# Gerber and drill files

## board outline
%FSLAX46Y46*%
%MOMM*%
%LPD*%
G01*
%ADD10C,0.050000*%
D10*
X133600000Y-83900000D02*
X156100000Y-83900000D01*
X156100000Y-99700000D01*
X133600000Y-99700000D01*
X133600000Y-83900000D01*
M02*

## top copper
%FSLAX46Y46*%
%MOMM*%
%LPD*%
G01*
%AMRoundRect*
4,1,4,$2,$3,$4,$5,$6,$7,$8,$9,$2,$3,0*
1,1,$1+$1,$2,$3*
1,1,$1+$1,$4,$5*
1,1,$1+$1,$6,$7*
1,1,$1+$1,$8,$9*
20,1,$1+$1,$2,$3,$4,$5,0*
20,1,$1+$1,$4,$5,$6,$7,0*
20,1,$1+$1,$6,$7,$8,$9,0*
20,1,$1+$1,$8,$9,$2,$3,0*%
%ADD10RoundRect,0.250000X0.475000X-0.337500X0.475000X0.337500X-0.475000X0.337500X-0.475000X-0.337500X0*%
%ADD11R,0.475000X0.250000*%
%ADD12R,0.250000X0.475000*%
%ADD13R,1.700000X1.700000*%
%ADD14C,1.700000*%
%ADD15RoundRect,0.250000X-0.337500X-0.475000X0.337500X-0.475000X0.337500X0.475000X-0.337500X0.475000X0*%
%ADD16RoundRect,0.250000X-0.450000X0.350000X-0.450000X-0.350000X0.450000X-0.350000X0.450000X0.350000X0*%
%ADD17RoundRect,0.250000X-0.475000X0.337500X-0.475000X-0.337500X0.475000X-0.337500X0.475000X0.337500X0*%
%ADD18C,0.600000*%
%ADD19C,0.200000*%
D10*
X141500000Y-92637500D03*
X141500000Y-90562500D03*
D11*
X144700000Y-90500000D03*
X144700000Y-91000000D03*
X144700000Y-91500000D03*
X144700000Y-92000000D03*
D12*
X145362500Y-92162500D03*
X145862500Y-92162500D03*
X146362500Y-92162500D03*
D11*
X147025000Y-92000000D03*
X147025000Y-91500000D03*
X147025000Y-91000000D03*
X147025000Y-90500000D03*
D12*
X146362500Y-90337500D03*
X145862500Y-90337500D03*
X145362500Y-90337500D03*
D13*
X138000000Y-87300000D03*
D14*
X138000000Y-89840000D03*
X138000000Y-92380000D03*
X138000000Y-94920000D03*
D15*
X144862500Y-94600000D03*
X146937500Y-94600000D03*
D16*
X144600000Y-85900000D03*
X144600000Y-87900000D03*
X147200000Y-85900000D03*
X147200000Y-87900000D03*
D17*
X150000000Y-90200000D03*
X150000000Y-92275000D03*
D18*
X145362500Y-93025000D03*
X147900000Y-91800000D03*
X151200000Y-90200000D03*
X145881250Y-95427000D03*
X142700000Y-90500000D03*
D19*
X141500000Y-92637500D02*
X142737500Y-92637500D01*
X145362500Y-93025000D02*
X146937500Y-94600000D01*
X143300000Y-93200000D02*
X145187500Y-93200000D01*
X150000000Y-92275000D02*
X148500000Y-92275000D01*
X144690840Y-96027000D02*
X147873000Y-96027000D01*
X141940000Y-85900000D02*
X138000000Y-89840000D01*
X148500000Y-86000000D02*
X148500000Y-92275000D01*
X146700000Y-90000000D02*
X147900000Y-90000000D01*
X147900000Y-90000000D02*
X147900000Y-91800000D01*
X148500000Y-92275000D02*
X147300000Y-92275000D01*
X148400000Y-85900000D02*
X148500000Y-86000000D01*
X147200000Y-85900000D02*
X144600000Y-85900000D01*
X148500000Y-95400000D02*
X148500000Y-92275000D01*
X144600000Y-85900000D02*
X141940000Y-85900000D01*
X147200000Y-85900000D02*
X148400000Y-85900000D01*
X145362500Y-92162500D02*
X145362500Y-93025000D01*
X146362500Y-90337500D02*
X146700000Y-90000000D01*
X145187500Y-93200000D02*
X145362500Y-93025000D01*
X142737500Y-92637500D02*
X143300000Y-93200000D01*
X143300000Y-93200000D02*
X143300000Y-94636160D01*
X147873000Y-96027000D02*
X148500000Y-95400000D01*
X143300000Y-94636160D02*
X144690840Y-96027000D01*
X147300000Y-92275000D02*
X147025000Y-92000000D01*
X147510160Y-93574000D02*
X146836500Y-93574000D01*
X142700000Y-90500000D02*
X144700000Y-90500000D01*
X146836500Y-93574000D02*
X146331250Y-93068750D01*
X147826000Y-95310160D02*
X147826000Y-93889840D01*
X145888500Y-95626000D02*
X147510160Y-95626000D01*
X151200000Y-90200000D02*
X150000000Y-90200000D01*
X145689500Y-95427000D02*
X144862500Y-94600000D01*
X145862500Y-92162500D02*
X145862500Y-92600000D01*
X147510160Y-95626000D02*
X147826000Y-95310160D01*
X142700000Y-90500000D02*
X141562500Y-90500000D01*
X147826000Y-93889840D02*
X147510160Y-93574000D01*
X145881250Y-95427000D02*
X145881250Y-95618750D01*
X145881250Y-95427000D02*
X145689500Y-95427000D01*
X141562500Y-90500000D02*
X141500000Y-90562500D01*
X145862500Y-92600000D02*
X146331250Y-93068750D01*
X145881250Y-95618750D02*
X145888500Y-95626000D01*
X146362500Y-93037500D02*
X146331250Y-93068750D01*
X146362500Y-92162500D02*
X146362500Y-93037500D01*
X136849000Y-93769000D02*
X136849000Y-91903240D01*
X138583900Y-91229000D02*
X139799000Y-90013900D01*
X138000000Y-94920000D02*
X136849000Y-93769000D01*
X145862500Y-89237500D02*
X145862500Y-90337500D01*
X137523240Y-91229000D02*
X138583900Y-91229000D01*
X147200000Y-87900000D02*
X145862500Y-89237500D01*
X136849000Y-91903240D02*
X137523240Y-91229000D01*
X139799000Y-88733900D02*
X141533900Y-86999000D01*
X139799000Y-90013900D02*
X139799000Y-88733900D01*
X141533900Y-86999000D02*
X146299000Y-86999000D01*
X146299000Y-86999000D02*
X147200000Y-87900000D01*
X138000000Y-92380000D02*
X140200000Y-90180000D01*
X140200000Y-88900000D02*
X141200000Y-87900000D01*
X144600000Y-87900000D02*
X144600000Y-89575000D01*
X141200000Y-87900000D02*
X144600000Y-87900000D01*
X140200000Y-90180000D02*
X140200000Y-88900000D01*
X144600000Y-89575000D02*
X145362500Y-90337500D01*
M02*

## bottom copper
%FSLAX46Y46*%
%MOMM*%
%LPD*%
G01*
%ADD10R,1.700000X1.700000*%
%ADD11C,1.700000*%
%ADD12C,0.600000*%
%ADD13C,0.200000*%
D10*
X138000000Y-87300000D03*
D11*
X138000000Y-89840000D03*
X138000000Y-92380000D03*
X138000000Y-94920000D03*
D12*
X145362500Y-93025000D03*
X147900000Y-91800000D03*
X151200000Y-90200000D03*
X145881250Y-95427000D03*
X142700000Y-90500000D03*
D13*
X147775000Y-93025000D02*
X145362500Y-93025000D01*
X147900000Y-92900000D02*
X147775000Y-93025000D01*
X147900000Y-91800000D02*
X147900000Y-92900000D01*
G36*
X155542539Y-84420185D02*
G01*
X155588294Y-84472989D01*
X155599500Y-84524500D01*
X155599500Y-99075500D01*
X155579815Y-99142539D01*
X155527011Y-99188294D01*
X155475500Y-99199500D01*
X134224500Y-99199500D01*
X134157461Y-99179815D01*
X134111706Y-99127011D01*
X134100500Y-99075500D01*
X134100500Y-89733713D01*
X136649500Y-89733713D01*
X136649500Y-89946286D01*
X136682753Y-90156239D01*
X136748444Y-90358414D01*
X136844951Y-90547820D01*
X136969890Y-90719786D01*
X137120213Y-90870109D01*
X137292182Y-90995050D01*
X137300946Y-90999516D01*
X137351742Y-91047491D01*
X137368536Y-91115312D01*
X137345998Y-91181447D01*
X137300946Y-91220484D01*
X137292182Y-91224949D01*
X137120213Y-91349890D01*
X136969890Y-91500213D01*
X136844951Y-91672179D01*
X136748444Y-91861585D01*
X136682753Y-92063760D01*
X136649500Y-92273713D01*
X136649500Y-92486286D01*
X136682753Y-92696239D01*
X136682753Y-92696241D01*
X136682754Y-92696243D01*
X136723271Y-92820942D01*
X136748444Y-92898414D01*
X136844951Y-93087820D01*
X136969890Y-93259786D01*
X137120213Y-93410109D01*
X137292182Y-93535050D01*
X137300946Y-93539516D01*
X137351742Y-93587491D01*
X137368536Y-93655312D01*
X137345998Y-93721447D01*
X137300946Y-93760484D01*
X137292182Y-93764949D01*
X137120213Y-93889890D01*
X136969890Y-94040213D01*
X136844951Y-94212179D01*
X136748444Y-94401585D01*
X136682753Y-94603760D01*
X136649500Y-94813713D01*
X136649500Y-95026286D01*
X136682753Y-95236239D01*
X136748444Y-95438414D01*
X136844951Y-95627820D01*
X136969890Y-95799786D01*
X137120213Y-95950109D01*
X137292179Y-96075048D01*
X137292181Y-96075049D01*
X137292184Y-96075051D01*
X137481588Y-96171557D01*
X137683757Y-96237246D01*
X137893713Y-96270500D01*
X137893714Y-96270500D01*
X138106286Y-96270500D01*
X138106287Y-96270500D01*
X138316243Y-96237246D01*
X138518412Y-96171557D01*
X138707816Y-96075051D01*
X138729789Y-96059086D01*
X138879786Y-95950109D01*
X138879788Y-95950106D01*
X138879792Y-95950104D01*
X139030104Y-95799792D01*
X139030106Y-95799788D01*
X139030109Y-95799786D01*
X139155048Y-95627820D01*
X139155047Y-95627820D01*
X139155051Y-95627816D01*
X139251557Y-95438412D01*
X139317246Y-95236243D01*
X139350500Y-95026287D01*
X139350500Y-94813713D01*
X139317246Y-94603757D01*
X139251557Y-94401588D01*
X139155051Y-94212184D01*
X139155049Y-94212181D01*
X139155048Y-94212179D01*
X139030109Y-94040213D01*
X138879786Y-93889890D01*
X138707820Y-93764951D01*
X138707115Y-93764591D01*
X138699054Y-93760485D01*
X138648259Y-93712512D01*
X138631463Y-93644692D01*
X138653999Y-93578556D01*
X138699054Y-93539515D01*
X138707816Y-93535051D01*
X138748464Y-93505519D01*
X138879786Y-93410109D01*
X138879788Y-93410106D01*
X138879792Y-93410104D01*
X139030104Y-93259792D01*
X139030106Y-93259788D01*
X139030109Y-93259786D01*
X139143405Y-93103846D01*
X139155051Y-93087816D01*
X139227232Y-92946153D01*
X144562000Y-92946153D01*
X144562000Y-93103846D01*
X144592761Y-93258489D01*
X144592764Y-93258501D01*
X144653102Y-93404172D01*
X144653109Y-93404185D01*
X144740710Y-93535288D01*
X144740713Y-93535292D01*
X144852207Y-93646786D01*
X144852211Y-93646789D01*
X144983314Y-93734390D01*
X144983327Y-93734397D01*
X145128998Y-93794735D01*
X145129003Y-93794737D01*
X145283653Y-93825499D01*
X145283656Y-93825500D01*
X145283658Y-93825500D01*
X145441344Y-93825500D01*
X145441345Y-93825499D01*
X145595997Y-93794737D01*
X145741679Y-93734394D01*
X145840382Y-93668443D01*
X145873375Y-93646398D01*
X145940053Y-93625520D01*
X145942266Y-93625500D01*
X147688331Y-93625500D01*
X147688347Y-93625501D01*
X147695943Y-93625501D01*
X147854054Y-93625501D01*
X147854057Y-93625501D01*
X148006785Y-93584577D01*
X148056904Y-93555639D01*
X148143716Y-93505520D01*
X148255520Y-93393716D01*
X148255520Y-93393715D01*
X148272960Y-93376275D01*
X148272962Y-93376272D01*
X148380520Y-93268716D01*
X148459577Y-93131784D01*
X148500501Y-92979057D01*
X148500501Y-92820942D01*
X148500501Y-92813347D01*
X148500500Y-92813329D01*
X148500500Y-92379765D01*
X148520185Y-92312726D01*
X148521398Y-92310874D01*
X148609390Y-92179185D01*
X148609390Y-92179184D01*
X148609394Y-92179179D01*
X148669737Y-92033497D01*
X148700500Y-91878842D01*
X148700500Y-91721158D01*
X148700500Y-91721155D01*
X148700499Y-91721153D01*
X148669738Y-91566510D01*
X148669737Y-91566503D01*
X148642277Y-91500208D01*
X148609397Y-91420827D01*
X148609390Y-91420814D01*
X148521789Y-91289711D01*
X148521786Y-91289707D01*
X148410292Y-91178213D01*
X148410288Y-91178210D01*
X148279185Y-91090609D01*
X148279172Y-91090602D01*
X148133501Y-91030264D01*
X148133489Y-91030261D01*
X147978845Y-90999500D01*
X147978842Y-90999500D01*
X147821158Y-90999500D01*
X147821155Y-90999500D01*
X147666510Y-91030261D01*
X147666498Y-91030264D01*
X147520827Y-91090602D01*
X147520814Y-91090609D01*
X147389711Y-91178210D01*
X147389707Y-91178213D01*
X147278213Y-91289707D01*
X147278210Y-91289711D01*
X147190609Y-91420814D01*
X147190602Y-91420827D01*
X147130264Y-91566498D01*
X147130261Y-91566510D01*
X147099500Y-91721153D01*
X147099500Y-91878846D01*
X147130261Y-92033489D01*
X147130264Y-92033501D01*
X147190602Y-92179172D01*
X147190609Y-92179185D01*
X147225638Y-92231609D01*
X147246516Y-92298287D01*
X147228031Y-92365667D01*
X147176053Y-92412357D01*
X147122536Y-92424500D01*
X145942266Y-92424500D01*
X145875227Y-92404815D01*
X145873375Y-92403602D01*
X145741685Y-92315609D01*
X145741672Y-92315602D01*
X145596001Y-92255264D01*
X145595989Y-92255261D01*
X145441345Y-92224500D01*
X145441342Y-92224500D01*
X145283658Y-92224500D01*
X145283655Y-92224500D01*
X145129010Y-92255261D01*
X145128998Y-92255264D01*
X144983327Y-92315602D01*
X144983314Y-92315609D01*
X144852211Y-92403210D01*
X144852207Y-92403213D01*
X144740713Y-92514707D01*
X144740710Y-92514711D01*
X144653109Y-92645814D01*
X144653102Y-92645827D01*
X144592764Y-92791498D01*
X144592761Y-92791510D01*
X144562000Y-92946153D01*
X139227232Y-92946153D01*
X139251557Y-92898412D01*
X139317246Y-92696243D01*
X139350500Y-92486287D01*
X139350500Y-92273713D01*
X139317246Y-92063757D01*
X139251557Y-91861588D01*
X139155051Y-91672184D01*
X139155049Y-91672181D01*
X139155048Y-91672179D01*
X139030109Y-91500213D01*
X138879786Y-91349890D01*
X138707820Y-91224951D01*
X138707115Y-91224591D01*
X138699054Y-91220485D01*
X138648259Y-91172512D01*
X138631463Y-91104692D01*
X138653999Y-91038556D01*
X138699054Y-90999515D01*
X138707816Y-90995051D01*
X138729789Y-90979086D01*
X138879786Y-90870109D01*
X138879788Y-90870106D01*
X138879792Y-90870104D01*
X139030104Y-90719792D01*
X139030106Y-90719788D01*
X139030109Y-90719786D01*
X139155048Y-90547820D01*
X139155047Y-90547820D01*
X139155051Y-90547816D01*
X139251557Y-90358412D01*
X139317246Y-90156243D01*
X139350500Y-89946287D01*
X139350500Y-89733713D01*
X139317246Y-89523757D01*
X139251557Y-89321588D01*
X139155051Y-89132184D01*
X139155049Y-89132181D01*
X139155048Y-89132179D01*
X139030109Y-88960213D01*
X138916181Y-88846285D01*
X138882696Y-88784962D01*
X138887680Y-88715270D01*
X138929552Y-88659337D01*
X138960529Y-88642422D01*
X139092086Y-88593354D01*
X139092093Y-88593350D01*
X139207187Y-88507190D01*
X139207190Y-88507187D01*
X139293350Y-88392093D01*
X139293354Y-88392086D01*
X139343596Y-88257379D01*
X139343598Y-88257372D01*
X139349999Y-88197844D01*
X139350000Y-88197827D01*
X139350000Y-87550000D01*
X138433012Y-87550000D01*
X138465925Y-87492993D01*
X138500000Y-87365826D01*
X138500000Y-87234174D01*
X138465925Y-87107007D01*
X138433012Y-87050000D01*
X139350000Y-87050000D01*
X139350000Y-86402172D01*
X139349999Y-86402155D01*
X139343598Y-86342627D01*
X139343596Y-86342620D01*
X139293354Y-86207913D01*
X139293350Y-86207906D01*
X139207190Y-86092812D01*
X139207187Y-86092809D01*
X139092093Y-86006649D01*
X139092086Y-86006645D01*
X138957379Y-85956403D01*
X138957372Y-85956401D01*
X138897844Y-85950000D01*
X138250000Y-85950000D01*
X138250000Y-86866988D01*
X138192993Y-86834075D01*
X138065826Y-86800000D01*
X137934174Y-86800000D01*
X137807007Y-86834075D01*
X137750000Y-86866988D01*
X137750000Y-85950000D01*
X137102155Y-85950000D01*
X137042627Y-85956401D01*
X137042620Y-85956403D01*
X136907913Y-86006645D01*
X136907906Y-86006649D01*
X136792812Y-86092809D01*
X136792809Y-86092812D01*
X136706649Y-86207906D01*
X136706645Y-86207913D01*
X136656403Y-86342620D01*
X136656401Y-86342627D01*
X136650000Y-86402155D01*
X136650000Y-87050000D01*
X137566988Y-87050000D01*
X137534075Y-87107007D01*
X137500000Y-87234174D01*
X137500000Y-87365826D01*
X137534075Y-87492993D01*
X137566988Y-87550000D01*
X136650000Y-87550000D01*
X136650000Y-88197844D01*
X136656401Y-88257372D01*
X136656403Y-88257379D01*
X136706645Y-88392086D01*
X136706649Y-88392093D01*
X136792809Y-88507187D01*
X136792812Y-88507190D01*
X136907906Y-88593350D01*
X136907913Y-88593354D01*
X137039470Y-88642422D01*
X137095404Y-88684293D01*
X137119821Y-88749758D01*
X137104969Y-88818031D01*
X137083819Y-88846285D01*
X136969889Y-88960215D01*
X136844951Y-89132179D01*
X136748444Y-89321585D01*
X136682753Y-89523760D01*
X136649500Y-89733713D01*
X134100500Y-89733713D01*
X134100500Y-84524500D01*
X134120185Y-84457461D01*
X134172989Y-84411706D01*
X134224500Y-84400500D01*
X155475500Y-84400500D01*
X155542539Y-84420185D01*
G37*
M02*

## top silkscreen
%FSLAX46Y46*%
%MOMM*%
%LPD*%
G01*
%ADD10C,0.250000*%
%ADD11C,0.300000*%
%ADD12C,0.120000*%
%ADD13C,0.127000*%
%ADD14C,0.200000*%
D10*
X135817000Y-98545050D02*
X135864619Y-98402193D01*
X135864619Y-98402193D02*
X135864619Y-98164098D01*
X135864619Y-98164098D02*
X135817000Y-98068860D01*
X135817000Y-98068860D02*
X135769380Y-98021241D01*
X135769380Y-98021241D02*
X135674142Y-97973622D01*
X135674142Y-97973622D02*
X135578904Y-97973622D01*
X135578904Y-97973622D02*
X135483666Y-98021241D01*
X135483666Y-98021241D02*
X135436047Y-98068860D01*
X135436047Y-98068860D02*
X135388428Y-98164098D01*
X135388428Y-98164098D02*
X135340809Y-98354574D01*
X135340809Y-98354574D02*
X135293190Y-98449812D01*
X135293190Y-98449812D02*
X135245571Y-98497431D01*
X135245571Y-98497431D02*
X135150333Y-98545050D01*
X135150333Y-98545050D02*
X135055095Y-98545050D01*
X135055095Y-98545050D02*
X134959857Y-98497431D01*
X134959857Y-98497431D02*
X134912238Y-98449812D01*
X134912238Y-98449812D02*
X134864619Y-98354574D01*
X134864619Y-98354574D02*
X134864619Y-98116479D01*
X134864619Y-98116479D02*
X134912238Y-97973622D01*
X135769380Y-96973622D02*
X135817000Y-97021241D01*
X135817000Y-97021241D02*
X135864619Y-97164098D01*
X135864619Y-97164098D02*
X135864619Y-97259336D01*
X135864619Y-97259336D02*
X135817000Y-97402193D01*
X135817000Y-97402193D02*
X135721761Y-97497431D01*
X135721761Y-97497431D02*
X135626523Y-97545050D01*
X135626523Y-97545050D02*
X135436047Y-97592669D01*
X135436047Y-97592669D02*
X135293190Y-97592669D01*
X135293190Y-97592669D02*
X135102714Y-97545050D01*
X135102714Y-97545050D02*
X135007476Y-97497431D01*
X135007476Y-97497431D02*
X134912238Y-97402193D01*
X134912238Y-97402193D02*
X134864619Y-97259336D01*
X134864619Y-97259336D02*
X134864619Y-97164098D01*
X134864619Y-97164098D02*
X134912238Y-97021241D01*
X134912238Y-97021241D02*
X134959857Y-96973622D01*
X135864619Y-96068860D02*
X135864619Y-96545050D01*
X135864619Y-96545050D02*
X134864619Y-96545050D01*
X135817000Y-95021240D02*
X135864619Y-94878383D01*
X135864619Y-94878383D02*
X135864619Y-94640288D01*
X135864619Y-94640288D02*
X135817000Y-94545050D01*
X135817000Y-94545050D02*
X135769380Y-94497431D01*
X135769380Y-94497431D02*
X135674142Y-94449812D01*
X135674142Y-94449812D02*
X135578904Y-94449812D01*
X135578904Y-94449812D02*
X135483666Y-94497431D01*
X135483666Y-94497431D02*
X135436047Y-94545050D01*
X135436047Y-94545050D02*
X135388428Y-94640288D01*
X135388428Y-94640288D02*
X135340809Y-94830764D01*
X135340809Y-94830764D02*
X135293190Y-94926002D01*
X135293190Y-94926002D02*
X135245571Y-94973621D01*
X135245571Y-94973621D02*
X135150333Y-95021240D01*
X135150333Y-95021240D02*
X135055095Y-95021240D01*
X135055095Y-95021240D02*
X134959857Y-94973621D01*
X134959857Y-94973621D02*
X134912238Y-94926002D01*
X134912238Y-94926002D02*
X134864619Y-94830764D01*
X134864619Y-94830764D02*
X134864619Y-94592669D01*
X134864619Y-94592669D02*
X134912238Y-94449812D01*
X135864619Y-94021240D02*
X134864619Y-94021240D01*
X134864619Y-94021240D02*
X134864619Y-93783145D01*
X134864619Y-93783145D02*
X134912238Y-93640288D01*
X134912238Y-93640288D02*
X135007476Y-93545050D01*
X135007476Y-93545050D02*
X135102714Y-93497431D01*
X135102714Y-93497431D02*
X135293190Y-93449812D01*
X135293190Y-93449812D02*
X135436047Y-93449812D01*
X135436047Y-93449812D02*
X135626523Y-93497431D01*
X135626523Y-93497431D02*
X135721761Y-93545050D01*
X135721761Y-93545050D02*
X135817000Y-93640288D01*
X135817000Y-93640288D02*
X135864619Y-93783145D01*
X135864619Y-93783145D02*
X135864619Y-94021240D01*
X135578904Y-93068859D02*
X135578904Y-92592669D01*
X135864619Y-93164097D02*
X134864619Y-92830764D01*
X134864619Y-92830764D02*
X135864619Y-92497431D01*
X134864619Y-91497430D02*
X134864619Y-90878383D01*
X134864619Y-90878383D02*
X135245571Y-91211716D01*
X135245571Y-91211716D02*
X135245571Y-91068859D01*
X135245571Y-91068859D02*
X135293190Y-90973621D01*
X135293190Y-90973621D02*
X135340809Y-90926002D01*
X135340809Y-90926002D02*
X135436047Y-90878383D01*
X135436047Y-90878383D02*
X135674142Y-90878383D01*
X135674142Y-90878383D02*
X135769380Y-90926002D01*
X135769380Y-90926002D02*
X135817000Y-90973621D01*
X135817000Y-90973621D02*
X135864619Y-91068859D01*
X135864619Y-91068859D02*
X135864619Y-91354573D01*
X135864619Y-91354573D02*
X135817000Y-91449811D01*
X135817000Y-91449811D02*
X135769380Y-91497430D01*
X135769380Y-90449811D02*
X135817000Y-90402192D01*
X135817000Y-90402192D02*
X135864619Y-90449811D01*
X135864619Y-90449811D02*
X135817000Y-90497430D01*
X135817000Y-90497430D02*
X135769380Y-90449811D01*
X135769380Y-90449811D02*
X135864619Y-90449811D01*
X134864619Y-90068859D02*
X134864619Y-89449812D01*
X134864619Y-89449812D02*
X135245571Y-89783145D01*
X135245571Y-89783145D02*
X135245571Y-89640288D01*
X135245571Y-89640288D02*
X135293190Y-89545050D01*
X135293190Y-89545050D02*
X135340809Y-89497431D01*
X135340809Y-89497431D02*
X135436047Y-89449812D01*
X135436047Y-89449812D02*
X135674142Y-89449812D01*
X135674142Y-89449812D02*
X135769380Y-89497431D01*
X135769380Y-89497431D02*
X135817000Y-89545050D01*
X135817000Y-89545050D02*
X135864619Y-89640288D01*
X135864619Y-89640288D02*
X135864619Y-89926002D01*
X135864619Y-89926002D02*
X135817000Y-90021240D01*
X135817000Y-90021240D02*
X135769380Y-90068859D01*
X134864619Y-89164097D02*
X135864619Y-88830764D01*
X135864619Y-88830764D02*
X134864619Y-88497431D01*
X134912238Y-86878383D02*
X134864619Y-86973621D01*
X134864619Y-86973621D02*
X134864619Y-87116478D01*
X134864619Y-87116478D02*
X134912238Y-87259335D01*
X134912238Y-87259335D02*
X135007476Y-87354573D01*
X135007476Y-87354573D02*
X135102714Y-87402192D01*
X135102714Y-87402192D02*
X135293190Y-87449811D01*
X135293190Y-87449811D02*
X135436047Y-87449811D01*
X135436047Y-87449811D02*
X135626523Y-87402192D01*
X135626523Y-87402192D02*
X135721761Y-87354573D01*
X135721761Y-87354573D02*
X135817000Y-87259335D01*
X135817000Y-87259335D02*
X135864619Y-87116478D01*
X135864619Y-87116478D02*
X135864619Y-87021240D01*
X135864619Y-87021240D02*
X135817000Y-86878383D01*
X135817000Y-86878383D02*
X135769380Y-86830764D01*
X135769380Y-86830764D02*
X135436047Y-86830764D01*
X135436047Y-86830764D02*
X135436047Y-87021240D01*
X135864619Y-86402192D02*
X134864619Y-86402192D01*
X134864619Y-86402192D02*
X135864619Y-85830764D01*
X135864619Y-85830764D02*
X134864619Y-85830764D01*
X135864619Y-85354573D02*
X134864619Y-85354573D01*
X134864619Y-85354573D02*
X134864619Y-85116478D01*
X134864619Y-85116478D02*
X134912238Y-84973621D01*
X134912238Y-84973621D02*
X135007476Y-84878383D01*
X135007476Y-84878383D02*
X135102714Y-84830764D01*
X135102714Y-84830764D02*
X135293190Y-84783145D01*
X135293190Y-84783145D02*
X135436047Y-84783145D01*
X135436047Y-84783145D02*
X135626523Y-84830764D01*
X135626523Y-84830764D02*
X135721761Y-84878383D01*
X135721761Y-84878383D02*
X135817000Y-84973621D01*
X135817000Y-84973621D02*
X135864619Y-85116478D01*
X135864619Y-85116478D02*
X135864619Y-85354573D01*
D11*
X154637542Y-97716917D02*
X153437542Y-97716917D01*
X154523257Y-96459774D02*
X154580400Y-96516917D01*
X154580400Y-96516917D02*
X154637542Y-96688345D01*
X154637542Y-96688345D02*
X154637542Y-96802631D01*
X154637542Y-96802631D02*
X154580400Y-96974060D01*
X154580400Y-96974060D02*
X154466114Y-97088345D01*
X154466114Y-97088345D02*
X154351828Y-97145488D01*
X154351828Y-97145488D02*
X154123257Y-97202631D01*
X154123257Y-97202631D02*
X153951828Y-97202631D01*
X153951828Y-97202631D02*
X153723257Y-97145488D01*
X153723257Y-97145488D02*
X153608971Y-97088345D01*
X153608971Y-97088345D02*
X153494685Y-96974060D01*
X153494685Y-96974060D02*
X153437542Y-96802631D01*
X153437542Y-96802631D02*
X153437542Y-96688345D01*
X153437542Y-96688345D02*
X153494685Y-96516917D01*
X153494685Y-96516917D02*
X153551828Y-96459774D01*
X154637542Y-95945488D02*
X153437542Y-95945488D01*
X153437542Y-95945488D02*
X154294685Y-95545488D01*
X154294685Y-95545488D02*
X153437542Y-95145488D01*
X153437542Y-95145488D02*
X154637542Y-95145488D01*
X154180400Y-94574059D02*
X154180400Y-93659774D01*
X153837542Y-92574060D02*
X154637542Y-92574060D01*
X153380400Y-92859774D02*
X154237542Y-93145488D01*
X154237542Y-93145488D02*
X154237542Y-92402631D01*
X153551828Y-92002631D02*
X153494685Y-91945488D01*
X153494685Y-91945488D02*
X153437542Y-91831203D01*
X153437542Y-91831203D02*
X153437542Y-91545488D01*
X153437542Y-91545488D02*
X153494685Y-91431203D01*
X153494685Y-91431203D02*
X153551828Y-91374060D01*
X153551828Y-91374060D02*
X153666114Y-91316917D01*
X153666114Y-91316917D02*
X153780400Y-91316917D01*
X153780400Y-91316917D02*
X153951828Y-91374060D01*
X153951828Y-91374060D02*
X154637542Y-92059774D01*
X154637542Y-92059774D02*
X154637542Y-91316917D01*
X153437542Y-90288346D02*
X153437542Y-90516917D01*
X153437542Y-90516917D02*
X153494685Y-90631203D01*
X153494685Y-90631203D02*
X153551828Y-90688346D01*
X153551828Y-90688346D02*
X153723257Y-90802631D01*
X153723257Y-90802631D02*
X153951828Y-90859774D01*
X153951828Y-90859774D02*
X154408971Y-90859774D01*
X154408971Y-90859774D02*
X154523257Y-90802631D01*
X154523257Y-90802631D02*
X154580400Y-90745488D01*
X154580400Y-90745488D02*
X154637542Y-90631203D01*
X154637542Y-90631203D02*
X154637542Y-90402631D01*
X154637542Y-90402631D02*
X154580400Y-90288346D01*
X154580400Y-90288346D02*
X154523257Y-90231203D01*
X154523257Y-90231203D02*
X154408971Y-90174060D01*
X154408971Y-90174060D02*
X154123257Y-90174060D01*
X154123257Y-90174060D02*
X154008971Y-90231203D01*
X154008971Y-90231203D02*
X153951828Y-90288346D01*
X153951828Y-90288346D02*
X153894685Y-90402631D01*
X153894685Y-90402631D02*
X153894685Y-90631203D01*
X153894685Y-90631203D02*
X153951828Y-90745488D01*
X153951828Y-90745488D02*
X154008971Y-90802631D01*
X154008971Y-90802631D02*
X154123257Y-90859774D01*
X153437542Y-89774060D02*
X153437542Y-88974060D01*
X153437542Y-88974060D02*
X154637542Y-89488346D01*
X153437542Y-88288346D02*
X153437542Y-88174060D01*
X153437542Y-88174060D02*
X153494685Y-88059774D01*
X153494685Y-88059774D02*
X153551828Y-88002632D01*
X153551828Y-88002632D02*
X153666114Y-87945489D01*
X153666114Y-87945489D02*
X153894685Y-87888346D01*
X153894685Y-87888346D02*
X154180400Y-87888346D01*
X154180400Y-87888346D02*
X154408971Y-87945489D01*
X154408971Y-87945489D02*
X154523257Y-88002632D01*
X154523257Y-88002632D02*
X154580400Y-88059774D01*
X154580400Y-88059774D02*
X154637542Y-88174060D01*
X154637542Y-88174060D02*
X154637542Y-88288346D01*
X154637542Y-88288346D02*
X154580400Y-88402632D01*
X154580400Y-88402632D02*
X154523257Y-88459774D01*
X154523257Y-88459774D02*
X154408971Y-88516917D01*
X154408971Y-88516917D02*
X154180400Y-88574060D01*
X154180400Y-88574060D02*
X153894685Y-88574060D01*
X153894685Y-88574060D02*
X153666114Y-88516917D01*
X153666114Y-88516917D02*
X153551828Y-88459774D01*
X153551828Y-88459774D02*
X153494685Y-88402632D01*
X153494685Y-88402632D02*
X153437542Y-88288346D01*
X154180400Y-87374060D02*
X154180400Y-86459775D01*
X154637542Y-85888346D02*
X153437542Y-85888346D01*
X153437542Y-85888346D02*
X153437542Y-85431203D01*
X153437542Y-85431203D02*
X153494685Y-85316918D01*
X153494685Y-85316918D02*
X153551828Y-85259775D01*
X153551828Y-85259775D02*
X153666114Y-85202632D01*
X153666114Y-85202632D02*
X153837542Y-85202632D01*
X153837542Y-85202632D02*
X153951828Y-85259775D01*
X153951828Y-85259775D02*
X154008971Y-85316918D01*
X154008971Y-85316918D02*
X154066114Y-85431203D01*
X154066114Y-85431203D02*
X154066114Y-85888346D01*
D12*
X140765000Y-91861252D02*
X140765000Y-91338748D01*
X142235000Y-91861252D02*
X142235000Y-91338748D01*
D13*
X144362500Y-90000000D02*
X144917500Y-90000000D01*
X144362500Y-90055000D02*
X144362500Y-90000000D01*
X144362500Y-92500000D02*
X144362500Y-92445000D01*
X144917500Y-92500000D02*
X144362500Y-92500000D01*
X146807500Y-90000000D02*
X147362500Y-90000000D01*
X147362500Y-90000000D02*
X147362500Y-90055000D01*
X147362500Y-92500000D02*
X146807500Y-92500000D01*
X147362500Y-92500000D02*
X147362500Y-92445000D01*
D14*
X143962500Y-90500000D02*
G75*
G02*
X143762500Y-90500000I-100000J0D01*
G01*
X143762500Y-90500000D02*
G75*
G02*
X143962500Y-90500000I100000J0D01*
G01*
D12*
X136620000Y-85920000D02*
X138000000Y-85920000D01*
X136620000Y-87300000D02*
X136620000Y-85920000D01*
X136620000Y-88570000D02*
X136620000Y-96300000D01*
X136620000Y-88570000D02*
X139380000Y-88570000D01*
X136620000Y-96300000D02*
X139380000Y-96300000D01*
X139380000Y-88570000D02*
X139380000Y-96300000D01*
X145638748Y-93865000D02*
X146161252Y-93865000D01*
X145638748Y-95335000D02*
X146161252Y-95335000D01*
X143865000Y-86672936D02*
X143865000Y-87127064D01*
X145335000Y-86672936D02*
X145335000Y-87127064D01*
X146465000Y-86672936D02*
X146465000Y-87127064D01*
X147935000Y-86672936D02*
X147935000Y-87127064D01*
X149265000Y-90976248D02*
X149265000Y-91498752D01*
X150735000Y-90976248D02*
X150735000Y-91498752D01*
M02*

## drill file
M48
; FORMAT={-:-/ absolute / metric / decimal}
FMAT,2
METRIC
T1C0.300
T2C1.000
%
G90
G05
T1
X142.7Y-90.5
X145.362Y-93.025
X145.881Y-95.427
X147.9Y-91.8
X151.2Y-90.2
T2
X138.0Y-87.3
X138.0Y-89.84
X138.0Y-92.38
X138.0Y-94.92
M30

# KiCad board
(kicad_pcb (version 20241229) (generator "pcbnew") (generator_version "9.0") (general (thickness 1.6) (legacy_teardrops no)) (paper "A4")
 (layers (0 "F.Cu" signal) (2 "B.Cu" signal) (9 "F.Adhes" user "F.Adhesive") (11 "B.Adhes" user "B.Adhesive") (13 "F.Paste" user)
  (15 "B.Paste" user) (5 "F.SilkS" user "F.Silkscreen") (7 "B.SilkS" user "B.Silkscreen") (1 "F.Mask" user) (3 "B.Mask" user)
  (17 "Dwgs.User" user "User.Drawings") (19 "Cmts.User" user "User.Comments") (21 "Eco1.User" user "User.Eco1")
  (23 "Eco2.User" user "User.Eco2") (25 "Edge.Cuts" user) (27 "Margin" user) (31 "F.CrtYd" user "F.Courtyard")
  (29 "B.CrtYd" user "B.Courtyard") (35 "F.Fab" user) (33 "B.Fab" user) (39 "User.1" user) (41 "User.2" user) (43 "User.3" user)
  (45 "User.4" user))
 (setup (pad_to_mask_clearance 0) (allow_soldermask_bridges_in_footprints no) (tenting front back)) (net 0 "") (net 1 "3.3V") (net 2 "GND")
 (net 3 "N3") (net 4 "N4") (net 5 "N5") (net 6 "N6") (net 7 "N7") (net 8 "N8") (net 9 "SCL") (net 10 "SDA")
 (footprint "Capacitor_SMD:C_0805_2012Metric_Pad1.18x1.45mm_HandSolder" (layer "F.Cu") (at 141.5 91.6 90)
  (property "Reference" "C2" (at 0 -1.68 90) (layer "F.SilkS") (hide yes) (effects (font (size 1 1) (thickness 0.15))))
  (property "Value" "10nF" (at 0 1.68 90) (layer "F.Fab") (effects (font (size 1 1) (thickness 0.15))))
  (fp_line (start -0.261252 -0.735) (end 0.261252 -0.735) (stroke (width 0.12) (type solid)) (layer "F.SilkS"))
  (fp_line (start -0.261252 0.735) (end 0.261252 0.735) (stroke (width 0.12) (type solid)) (layer "F.SilkS"))
  (pad "1" smd roundrect (at -1.0375 0 90) (size 1.175 1.45) (layers "F.Cu" "F.Mask" "F.Paste") (roundrect_rratio 0.212766) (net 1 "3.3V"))
  (pad "2" smd roundrect (at 1.0375 0 90) (size 1.175 1.45) (layers "F.Cu" "F.Mask" "F.Paste") (roundrect_rratio 0.212766) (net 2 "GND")))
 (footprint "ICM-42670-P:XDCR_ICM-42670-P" (layer "F.Cu") (at 145.8625 91.25)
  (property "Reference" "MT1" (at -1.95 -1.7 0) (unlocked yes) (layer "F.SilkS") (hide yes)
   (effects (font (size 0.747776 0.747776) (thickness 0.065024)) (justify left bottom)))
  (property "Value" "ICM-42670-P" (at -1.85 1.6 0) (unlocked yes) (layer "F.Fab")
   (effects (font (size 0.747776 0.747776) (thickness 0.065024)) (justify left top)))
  (fp_line (start -1.5 -1.25) (end -0.945 -1.25) (stroke (width 0.127) (type solid)) (layer "F.SilkS"))
  (fp_line (start -1.5 -1.195) (end -1.5 -1.25) (stroke (width 0.127) (type solid)) (layer "F.SilkS"))
  (fp_line (start -1.5 1.25) (end -1.5 1.195) (stroke (width 0.127) (type solid)) (layer "F.SilkS"))
  (fp_line (start -0.945 1.25) (end -1.5 1.25) (stroke (width 0.127) (type solid)) (layer "F.SilkS"))
  (fp_line (start 0.945 -1.25) (end 1.5 -1.25) (stroke (width 0.127) (type solid)) (layer "F.SilkS"))
  (fp_line (start 1.5 -1.25) (end 1.5 -1.195) (stroke (width 0.127) (type solid)) (layer "F.SilkS"))
  (fp_line (start 1.5 1.25) (end 0.945 1.25) (stroke (width 0.127) (type solid)) (layer "F.SilkS"))
  (fp_line (start 1.5 1.25) (end 1.5 1.195) (stroke (width 0.127) (type solid)) (layer "F.SilkS"))
  (fp_circle (center -2 -0.75) (end -1.9 -0.75) (stroke (width 0.2) (type solid)) (fill no) (layer "F.SilkS"))
  (pad "1" smd rect (at -1.1625 -0.75) (size 0.475 0.25) (layers "F.Cu") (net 2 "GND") (solder_mask_margin 0.1016) (solder_paste_margin 0)
   (thermal_bridge_angle 0))
  (pad "2" smd rect (at -1.1625 -0.25) (size 0.475 0.25) (layers "F.Cu") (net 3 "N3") (solder_mask_margin 0.1016) (solder_paste_margin 0)
   (thermal_bridge_angle 0))
  (pad "3" smd rect (at -1.1625 0.25) (size 0.475 0.25) (layers "F.Cu") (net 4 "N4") (solder_mask_margin 0.1016) (solder_paste_margin 0)
   (thermal_bridge_angle 0))
  (pad "4" smd rect (at -1.1625 0.75) (size 0.475 0.25) (layers "F.Cu") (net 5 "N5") (solder_mask_margin 0.1016) (solder_paste_margin 0)
   (thermal_bridge_angle 0))
  (pad "5" smd rect (at -0.5 0.9125) (size 0.25 0.475) (layers "F.Cu") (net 1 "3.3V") (solder_mask_margin 0.1016) (solder_paste_margin 0)
   (thermal_bridge_angle 0))
  (pad "6" smd rect (at 0 0.9125) (size 0.25 0.475) (layers "F.Cu") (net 2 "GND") (solder_mask_margin 0.1016) (solder_paste_margin 0)
   (thermal_bridge_angle 0))
  (pad "7" smd rect (at 0.5 0.9125) (size 0.25 0.475) (layers "F.Cu") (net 2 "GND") (solder_mask_margin 0.1016) (solder_paste_margin 0)
   (thermal_bridge_angle 0))
  (pad "8" smd rect (at 1.1625 0.75) (size 0.475 0.25) (layers "F.Cu") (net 1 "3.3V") (solder_mask_margin 0.1016) (solder_paste_margin 0)
   (thermal_bridge_angle 0))
  (pad "9" smd rect (at 1.1625 0.25) (size 0.475 0.25) (layers "F.Cu") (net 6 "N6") (solder_mask_margin 0.1016) (solder_paste_margin 0)
   (thermal_bridge_angle 0))
  (pad "10" smd rect (at 1.1625 -0.25) (size 0.475 0.25) (layers "F.Cu") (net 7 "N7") (solder_mask_margin 0.1016) (solder_paste_margin 0)
   (thermal_bridge_angle 0))
  (pad "11" smd rect (at 1.1625 -0.75) (size 0.475 0.25) (layers "F.Cu") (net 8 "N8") (solder_mask_margin 0.1016) (solder_paste_margin 0)
   (thermal_bridge_angle 0))
  (pad "12" smd rect (at 0.5 -0.9125) (size 0.25 0.475) (layers "F.Cu") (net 1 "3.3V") (solder_mask_margin 0.1016) (solder_paste_margin 0)
   (thermal_bridge_angle 0))
  (pad "13" smd rect (at 0 -0.9125) (size 0.25 0.475) (layers "F.Cu") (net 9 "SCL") (solder_mask_margin 0.1016) (solder_paste_margin 0)
   (thermal_bridge_angle 0))
  (pad "14" smd rect (at -0.5 -0.9125) (size 0.25 0.475) (layers "F.Cu") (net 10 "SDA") (solder_mask_margin 0.1016) (solder_paste_margin 0)
   (thermal_bridge_angle 0))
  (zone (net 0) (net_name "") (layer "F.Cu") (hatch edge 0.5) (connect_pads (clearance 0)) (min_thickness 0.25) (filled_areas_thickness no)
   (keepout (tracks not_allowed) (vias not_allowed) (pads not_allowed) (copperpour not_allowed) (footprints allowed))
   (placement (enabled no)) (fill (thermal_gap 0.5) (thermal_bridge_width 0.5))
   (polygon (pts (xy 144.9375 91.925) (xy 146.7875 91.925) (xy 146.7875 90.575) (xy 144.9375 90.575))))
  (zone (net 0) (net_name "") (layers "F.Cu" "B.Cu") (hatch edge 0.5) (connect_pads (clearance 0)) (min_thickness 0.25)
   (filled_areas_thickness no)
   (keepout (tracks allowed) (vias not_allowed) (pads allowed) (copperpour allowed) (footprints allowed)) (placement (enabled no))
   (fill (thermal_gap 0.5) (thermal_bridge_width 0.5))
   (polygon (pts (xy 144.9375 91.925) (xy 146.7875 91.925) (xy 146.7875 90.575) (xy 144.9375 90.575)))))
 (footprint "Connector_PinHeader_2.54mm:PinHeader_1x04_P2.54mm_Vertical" (layer "F.Cu") (at 138 87.3)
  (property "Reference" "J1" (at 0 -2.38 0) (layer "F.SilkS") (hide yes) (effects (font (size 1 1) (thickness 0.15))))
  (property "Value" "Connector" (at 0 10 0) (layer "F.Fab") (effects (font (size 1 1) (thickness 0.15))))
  (fp_line (start -1.38 -1.38) (end 0 -1.38) (stroke (width 0.12) (type solid)) (layer "F.SilkS"))
  (fp_line (start -1.38 0) (end -1.38 -1.38) (stroke (width 0.12) (type solid)) (layer "F.SilkS"))
  (fp_line (start -1.38 1.27) (end -1.38 9) (stroke (width 0.12) (type solid)) (layer "F.SilkS"))
  (fp_line (start -1.38 1.27) (end 1.38 1.27) (stroke (width 0.12) (type solid)) (layer "F.SilkS"))
  (fp_line (start -1.38 9) (end 1.38 9) (stroke (width 0.12) (type solid)) (layer "F.SilkS"))
  (fp_line (start 1.38 1.27) (end 1.38 9) (stroke (width 0.12) (type solid)) (layer "F.SilkS"))
  (pad "1" thru_hole rect (at 0 0) (size 1.7 1.7) (drill 1) (layers "*.Cu" "*.Mask") (remove_unused_layers no) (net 2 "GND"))
  (pad "2" thru_hole circle (at 0 2.54) (size 1.7 1.7) (drill 1) (layers "*.Cu" "*.Mask") (remove_unused_layers no) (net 1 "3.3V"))
  (pad "3" thru_hole circle (at 0 5.08) (size 1.7 1.7) (drill 1) (layers "*.Cu" "*.Mask") (remove_unused_layers no) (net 10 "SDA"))
  (pad "4" thru_hole circle (at 0 7.62) (size 1.7 1.7) (drill 1) (layers "*.Cu" "*.Mask") (remove_unused_layers no) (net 9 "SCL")))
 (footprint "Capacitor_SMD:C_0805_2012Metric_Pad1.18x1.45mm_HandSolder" (layer "F.Cu") (at 145.9 94.6)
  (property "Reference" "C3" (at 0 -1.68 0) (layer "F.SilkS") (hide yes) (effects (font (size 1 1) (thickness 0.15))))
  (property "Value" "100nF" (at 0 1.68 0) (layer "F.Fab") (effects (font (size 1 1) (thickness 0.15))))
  (fp_line (start -0.261252 -0.735) (end 0.261252 -0.735) (stroke (width 0.12) (type solid)) (layer "F.SilkS"))
  (fp_line (start -0.261252 0.735) (end 0.261252 0.735) (stroke (width 0.12) (type solid)) (layer "F.SilkS"))
  (pad "1" smd roundrect (at -1.0375 0) (size 1.175 1.45) (layers "F.Cu" "F.Mask" "F.Paste") (roundrect_rratio 0.212766) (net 2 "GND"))
  (pad "2" smd roundrect (at 1.0375 0) (size 1.175 1.45) (layers "F.Cu" "F.Mask" "F.Paste") (roundrect_rratio 0.212766) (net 1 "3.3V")))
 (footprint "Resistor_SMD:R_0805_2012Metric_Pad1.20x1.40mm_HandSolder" (layer "F.Cu") (at 144.6 86.9 -90)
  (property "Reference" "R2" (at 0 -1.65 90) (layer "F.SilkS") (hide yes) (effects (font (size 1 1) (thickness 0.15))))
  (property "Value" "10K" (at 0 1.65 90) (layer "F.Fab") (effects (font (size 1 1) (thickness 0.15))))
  (fp_line (start -0.227064 0.735) (end 0.227064 0.735) (stroke (width 0.12) (type solid)) (layer "F.SilkS"))
  (fp_line (start -0.227064 -0.735) (end 0.227064 -0.735) (stroke (width 0.12) (type solid)) (layer "F.SilkS"))
  (pad "1" smd roundrect (at -1 0 270) (size 1.2 1.4) (layers "F.Cu" "F.Mask" "F.Paste") (roundrect_rratio 0.208333) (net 1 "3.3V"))
  (pad "2" smd roundrect (at 1 0 270) (size 1.2 1.4) (layers "F.Cu" "F.Mask" "F.Paste") (roundrect_rratio 0.208333) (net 10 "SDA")))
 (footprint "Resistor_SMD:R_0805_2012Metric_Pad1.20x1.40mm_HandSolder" (layer "F.Cu") (at 147.2 86.9 -90)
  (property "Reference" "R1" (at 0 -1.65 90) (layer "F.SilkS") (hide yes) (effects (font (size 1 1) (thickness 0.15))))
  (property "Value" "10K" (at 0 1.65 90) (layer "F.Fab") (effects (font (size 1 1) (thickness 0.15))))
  (fp_line (start -0.227064 0.735) (end 0.227064 0.735) (stroke (width 0.12) (type solid)) (layer "F.SilkS"))
  (fp_line (start -0.227064 -0.735) (end 0.227064 -0.735) (stroke (width 0.12) (type solid)) (layer "F.SilkS"))
  (pad "1" smd roundrect (at -1 0 270) (size 1.2 1.4) (layers "F.Cu" "F.Mask" "F.Paste") (roundrect_rratio 0.208333) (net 1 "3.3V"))
  (pad "2" smd roundrect (at 1 0 270) (size 1.2 1.4) (layers "F.Cu" "F.Mask" "F.Paste") (roundrect_rratio 0.208333) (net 9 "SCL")))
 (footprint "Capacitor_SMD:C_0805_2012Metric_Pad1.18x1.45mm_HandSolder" (layer "F.Cu") (at 150 91.2375 -90)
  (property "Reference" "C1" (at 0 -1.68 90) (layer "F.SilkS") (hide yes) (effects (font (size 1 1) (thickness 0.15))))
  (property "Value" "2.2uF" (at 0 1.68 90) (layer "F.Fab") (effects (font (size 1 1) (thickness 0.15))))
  (fp_line (start -0.261252 0.735) (end 0.261252 0.735) (stroke (width 0.12) (type solid)) (layer "F.SilkS"))
  (fp_line (start -0.261252 -0.735) (end 0.261252 -0.735) (stroke (width 0.12) (type solid)) (layer "F.SilkS"))
  (pad "1" smd roundrect (at -1.0375 0 270) (size 1.175 1.45) (layers "F.Cu" "F.Mask" "F.Paste") (roundrect_rratio 0.212766) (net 2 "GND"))
  (pad "2" smd roundrect (at 1.0375 0 270) (size 1.175 1.45) (layers "F.Cu" "F.Mask" "F.Paste") (roundrect_rratio 0.212766) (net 1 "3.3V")))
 (gr_rect (start 133.6 83.9) (end 156.1 99.7) (stroke (width 0.05) (type default)) (fill no) (layer "Edge.Cuts"))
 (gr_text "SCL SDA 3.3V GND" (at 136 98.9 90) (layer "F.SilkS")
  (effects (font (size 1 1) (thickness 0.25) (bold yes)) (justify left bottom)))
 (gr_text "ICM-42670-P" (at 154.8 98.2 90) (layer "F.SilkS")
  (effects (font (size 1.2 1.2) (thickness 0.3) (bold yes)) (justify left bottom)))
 (segment (start 141.5 92.6375) (end 142.7375 92.6375) (width 0.2) (layer "F.Cu") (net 1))
 (segment (start 145.3625 93.025) (end 146.9375 94.6) (width 0.2) (layer "F.Cu") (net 1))
 (segment (start 143.3 93.2) (end 145.1875 93.2) (width 0.2) (layer "F.Cu") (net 1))
 (segment (start 150 92.275) (end 148.5 92.275) (width 0.2) (layer "F.Cu") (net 1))
 (segment (start 144.69084 96.027) (end 147.873 96.027) (width 0.2) (layer "F.Cu") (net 1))
 (segment (start 141.94 85.9) (end 138 89.84) (width 0.2) (layer "F.Cu") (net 1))
 (segment (start 148.5 86) (end 148.5 92.275) (width 0.2) (layer "F.Cu") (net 1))
 (segment (start 146.7 90) (end 147.9 90) (width 0.2) (layer "F.Cu") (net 1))
 (segment (start 147.9 90) (end 147.9 91.8) (width 0.2) (layer "F.Cu") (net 1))
 (segment (start 148.5 92.275) (end 147.3 92.275) (width 0.2) (layer "F.Cu") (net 1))
 (segment (start 148.4 85.9) (end 148.5 86) (width 0.2) (layer "F.Cu") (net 1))
 (segment (start 147.2 85.9) (end 144.6 85.9) (width 0.2) (layer "F.Cu") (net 1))
 (segment (start 148.5 95.4) (end 148.5 92.275) (width 0.2) (layer "F.Cu") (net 1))
 (segment (start 144.6 85.9) (end 141.94 85.9) (width 0.2) (layer "F.Cu") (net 1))
 (segment (start 147.2 85.9) (end 148.4 85.9) (width 0.2) (layer "F.Cu") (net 1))
 (segment (start 145.3625 92.1625) (end 145.3625 93.025) (width 0.2) (layer "F.Cu") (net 1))
 (segment (start 146.3625 90.3375) (end 146.7 90) (width 0.2) (layer "F.Cu") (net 1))
 (segment (start 145.1875 93.2) (end 145.3625 93.025) (width 0.2) (layer "F.Cu") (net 1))
 (segment (start 142.7375 92.6375) (end 143.3 93.2) (width 0.2) (layer "F.Cu") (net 1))
 (segment (start 143.3 93.2) (end 143.3 94.63616) (width 0.2) (layer "F.Cu") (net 1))
 (segment (start 147.873 96.027) (end 148.5 95.4) (width 0.2) (layer "F.Cu") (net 1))
 (segment (start 143.3 94.63616) (end 144.69084 96.027) (width 0.2) (layer "F.Cu") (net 1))
 (segment (start 147.3 92.275) (end 147.025 92) (width 0.2) (layer "F.Cu") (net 1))
 (via (at 145.3625 93.025) (size 0.6) (drill 0.3) (layers "F.Cu" "B.Cu") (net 1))
 (via (at 147.9 91.8) (size 0.6) (drill 0.3) (layers "F.Cu" "B.Cu") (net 1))
 (segment (start 147.775 93.025) (end 145.3625 93.025) (width 0.2) (layer "B.Cu") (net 1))
 (segment (start 147.9 92.9) (end 147.775 93.025) (width 0.2) (layer "B.Cu") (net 1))
 (segment (start 147.9 91.8) (end 147.9 92.9) (width 0.2) (layer "B.Cu") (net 1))
 (segment (start 147.51016 93.574) (end 146.8365 93.574) (width 0.2) (layer "F.Cu") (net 2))
 (segment (start 142.7 90.5) (end 144.7 90.5) (width 0.2) (layer "F.Cu") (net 2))
 (segment (start 146.8365 93.574) (end 146.33125 93.06875) (width 0.2) (layer "F.Cu") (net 2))
 (segment (start 147.826 95.31016) (end 147.826 93.88984) (width 0.2) (layer "F.Cu") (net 2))
 (segment (start 145.8885 95.626) (end 147.51016 95.626) (width 0.2) (layer "F.Cu") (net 2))
 (segment (start 151.2 90.2) (end 150 90.2) (width 0.2) (layer "F.Cu") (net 2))
 (segment (start 145.6895 95.427) (end 144.8625 94.6) (width 0.2) (layer "F.Cu") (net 2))
 (segment (start 145.8625 92.1625) (end 145.8625 92.6) (width 0.2) (layer "F.Cu") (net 2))
 (segment (start 147.51016 95.626) (end 147.826 95.31016) (width 0.2) (layer "F.Cu") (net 2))
 (segment (start 142.7 90.5) (end 141.5625 90.5) (width 0.2) (layer "F.Cu") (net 2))
 (segment (start 147.826 93.88984) (end 147.51016 93.574) (width 0.2) (layer "F.Cu") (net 2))
 (segment (start 145.88125 95.427) (end 145.88125 95.61875) (width 0.2) (layer "F.Cu") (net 2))
 (segment (start 145.88125 95.427) (end 145.6895 95.427) (width 0.2) (layer "F.Cu") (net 2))
 (segment (start 141.5625 90.5) (end 141.5 90.5625) (width 0.2) (layer "F.Cu") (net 2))
 (segment (start 145.8625 92.6) (end 146.33125 93.06875) (width 0.2) (layer "F.Cu") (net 2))
 (segment (start 145.88125 95.61875) (end 145.8885 95.626) (width 0.2) (layer "F.Cu") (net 2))
 (segment (start 146.3625 93.0375) (end 146.33125 93.06875) (width 0.2) (layer "F.Cu") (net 2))
 (segment (start 146.3625 92.1625) (end 146.3625 93.0375) (width 0.2) (layer "F.Cu") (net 2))
 (via (at 151.2 90.2) (size 0.6) (drill 0.3) (layers "F.Cu" "B.Cu") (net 2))
 (via (at 145.88125 95.427) (size 0.6) (drill 0.3) (layers "F.Cu" "B.Cu") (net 2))
 (via (at 142.7 90.5) (size 0.6) (drill 0.3) (layers "F.Cu" "B.Cu") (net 2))
 (segment (start 136.849 93.769) (end 136.849 91.90324) (width 0.2) (layer "F.Cu") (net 9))
 (segment (start 138.5839 91.229) (end 139.799 90.0139) (width 0.2) (layer "F.Cu") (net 9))
 (segment (start 138 94.92) (end 136.849 93.769) (width 0.2) (layer "F.Cu") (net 9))
 (segment (start 145.8625 89.2375) (end 145.8625 90.3375) (width 0.2) (layer "F.Cu") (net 9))
 (segment (start 137.52324 91.229) (end 138.5839 91.229) (width 0.2) (layer "F.Cu") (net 9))
 (segment (start 147.2 87.9) (end 145.8625 89.2375) (width 0.2) (layer "F.Cu") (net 9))
 (segment (start 136.849 91.90324) (end 137.52324 91.229) (width 0.2) (layer "F.Cu") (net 9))
 (segment (start 139.799 88.7339) (end 141.5339 86.999) (width 0.2) (layer "F.Cu") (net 9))
 (segment (start 139.799 90.0139) (end 139.799 88.7339) (width 0.2) (layer "F.Cu") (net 9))
 (segment (start 141.5339 86.999) (end 146.299 86.999) (width 0.2) (layer "F.Cu") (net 9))
 (segment (start 146.299 86.999) (end 147.2 87.9) (width 0.2) (layer "F.Cu") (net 9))
 (segment (start 138 92.38) (end 140.2 90.18) (width 0.2) (layer "F.Cu") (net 10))
 (segment (start 140.2 88.9) (end 141.2 87.9) (width 0.2) (layer "F.Cu") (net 10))
 (segment (start 144.6 87.9) (end 144.6 89.575) (width 0.2) (layer "F.Cu") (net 10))
 (segment (start 141.2 87.9) (end 144.6 87.9) (width 0.2) (layer "F.Cu") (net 10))
 (segment (start 140.2 90.18) (end 140.2 88.9) (width 0.2) (layer "F.Cu") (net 10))
 (segment (start 144.6 89.575) (end 145.3625 90.3375) (width 0.2) (layer "F.Cu") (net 10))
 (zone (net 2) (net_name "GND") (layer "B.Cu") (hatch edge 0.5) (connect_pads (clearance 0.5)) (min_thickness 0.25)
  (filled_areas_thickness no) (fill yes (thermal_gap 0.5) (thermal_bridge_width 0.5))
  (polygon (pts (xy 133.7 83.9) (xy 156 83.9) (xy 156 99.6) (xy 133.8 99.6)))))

